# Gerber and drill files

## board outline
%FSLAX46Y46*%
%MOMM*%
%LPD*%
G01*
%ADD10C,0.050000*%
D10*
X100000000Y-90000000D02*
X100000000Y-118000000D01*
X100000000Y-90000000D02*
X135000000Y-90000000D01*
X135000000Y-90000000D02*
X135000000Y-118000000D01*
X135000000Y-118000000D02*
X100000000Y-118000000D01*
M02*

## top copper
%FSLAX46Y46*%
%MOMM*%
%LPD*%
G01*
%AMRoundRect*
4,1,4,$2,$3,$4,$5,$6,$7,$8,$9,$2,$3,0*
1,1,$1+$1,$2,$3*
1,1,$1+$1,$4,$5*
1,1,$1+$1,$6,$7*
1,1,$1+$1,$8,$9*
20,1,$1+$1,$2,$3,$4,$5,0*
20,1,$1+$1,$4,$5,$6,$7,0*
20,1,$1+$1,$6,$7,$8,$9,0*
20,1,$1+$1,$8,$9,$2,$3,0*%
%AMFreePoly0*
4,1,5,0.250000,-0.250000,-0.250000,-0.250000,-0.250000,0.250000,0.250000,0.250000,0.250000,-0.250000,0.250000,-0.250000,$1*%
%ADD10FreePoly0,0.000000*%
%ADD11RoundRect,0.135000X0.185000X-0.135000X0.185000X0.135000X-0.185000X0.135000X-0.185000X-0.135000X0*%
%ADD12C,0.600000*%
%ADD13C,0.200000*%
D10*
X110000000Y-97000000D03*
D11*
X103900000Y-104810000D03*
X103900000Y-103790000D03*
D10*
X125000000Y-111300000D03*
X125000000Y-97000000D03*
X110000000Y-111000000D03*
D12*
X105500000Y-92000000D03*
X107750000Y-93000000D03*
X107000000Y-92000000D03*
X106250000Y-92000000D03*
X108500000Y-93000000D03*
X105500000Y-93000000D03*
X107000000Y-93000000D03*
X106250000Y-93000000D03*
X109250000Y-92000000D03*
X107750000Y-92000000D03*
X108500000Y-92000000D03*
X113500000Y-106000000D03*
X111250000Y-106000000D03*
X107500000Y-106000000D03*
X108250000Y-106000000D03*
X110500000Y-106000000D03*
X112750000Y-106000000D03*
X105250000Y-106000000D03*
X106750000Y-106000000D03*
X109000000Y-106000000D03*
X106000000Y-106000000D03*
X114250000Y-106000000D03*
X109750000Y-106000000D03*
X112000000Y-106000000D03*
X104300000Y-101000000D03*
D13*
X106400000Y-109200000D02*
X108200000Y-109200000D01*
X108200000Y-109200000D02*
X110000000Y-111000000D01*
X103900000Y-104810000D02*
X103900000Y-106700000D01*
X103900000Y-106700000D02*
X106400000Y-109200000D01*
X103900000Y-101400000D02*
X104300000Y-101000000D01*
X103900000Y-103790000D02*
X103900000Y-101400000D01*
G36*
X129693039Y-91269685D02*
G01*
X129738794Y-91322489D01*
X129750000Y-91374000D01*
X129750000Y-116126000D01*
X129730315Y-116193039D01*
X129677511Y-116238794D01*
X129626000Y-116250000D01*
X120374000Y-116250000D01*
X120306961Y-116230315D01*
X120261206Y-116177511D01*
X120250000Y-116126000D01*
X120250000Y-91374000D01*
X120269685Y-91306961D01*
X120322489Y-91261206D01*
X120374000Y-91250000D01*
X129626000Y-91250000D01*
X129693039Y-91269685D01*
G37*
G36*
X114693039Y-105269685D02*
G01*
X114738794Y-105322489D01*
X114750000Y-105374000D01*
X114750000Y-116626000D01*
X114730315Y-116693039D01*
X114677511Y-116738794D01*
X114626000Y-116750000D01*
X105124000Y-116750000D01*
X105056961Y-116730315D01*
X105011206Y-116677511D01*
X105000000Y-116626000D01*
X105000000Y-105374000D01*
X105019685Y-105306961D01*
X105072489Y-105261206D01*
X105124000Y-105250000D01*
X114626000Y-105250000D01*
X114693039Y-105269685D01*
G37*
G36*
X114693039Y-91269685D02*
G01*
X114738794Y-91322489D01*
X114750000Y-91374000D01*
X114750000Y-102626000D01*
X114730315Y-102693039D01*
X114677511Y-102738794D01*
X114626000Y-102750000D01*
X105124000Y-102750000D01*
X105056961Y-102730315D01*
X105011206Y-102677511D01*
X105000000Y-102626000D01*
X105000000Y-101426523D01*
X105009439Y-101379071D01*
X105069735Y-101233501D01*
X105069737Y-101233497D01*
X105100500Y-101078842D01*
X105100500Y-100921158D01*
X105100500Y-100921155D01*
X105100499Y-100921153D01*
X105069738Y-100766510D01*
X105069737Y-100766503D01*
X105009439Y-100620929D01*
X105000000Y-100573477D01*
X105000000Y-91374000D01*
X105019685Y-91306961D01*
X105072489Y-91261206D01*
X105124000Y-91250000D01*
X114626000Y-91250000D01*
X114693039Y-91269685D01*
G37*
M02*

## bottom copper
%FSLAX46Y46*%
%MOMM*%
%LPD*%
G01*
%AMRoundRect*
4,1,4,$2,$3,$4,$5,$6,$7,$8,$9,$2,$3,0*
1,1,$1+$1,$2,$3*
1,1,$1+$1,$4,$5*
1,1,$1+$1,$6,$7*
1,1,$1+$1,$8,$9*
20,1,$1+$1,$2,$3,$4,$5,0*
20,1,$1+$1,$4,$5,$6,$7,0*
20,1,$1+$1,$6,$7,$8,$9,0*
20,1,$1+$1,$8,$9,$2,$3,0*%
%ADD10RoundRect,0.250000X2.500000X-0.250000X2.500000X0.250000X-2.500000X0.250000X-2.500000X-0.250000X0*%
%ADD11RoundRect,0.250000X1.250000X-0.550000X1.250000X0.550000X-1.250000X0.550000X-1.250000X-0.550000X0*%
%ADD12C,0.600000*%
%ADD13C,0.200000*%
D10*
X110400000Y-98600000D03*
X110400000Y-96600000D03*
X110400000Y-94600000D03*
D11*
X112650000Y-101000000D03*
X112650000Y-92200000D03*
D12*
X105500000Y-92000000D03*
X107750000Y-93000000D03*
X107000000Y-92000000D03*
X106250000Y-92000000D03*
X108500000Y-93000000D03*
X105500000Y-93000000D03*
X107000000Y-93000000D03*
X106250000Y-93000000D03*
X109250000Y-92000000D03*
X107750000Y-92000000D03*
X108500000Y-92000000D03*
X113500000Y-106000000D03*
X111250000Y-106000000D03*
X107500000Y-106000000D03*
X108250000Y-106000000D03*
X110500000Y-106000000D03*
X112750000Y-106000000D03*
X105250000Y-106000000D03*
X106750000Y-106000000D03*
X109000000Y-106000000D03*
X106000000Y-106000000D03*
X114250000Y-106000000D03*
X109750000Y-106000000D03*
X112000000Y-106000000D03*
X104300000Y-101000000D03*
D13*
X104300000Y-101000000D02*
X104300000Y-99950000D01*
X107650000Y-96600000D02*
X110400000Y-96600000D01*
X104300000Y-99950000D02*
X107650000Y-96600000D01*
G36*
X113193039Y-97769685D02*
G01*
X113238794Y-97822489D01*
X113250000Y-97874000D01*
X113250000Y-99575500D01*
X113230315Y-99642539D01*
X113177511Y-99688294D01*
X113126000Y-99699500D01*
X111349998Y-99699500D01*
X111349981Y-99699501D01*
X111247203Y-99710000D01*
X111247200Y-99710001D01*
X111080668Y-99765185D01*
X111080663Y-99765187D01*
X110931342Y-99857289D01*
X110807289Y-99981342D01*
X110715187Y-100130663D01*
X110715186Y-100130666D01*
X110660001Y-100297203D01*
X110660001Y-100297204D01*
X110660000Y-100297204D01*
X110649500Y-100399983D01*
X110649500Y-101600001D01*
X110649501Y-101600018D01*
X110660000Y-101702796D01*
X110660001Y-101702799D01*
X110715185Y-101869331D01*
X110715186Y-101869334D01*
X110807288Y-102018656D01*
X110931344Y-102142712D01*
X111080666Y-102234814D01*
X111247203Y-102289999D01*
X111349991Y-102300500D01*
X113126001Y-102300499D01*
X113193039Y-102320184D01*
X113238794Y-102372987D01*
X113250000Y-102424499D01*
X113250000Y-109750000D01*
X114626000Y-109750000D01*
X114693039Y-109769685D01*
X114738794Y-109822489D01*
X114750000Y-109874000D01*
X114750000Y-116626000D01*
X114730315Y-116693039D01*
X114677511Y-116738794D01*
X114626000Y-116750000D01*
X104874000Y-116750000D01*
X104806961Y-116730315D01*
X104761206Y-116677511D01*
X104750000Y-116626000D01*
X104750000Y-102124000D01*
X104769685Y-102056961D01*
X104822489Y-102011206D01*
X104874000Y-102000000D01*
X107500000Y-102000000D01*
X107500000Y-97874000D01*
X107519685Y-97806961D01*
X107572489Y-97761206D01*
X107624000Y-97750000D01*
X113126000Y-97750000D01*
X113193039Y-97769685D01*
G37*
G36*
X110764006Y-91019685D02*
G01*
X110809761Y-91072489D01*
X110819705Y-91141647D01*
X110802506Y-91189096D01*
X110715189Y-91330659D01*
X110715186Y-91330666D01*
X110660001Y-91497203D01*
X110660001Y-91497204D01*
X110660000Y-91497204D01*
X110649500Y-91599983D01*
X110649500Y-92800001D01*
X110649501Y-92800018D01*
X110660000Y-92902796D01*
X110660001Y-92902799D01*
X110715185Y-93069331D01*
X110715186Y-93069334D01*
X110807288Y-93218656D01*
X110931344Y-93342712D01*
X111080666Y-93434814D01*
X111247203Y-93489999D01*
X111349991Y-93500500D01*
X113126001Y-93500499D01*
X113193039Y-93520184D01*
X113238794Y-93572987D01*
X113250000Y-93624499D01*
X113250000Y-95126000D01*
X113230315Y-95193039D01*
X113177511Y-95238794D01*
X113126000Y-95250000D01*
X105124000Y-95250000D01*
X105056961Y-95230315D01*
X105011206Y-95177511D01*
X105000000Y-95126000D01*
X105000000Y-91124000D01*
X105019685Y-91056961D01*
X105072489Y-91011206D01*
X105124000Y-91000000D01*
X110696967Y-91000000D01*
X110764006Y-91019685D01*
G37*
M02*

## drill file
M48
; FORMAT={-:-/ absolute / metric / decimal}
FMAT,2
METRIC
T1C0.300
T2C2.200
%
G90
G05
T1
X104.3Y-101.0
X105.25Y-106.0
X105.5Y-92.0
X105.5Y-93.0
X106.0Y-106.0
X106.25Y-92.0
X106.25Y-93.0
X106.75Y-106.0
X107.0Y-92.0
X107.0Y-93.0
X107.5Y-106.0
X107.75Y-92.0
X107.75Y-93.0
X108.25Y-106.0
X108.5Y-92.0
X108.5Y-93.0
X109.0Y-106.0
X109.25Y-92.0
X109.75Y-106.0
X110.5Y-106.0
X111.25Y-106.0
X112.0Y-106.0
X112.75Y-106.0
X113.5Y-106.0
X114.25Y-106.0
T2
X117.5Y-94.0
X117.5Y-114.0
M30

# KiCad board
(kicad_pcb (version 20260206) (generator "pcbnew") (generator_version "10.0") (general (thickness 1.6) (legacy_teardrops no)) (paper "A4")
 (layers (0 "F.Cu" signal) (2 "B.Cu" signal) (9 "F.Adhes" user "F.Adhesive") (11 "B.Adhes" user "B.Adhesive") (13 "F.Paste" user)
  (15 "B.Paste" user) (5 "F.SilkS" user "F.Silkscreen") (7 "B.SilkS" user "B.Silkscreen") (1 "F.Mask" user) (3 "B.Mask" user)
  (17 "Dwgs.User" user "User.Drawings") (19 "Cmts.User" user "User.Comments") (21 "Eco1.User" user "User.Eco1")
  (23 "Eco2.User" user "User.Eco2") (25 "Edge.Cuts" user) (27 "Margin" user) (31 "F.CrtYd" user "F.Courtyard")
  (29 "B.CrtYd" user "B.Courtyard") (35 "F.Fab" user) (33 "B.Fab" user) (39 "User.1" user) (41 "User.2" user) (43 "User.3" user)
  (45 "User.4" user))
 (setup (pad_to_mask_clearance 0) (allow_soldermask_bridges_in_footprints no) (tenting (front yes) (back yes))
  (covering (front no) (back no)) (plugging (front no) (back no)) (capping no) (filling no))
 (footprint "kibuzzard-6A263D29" (layer "F.Cu") (at 132.5 92.25)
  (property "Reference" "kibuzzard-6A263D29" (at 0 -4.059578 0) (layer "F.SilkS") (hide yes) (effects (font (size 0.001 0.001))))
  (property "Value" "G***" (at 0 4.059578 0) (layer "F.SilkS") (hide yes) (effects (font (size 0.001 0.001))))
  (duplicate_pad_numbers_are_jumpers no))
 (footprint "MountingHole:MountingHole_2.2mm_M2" (layer "F.Cu") (at 117.5 94)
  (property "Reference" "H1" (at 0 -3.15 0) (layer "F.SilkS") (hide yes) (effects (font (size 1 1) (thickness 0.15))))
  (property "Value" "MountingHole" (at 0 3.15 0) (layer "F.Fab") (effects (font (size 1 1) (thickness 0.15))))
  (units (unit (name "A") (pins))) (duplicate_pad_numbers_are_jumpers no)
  (pad "" np_thru_hole circle (at 0 0) (size 2.2 2.2) (drill 2.2) (layers "*.Cu" "*.Mask")))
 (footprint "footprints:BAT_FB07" (layer "F.Cu") (at 110 97)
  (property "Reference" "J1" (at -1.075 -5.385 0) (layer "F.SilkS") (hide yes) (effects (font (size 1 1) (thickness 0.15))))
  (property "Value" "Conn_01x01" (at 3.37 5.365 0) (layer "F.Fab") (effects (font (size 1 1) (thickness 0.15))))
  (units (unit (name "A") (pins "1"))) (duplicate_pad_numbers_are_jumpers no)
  (pad "1" smd custom (at 0 0) (size 0.5 0.5) (layers "F.Cu") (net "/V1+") (options (clearance outline) (anchor rect)) (primitives)))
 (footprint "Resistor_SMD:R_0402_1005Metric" (layer "F.Cu") (at 103.9 104.3 90)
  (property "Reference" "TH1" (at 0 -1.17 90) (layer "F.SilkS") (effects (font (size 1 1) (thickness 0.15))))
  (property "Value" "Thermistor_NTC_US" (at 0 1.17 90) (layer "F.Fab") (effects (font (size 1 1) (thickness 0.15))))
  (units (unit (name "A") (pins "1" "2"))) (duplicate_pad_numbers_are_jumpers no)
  (pad "1" smd roundrect (at -0.51 0 90) (size 0.54 0.64) (layers "F.Cu" "F.Mask" "F.Paste") (roundrect_rratio 0.25) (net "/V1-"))
  (pad "2" smd roundrect (at 0.51 0 90) (size 0.54 0.64) (layers "F.Cu" "F.Mask" "F.Paste") (roundrect_rratio 0.25) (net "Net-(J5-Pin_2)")))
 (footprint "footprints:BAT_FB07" (layer "F.Cu") (at 125 111.3)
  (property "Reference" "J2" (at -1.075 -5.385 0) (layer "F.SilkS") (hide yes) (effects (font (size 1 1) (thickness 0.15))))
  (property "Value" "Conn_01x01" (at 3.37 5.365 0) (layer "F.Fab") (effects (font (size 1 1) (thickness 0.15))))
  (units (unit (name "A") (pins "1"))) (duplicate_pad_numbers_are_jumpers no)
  (pad "1" smd custom (at 0 0) (size 0.5 0.5) (layers "F.Cu") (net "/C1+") (options (clearance outline) (anchor rect)) (primitives)))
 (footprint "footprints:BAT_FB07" (layer "F.Cu") (at 125 97)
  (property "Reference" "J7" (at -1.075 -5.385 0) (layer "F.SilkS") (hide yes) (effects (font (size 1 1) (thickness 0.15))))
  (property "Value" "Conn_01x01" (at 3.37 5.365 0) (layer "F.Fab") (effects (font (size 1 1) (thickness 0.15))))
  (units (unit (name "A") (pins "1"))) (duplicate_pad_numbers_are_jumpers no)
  (pad "1" smd custom (at 0 0) (size 0.5 0.5) (layers "F.Cu") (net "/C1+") (options (clearance outline) (anchor rect)) (primitives)))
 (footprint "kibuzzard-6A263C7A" (layer "F.Cu") (at 102.5 93)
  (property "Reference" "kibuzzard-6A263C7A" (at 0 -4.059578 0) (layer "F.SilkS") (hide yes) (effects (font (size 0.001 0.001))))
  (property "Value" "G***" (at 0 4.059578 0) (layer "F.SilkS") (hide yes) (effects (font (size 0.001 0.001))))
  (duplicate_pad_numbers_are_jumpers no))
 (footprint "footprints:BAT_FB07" (layer "F.Cu") (at 110 111)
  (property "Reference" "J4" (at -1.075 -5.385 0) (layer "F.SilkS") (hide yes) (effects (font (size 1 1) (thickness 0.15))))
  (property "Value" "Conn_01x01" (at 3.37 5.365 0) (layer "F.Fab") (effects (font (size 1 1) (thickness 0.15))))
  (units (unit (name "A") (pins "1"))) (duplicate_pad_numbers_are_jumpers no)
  (pad "1" smd custom (at 0 0) (size 0.5 0.5) (layers "F.Cu") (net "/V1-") (options (clearance outline) (anchor rect)) (primitives)))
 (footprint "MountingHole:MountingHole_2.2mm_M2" (layer "F.Cu") (at 117.5 114)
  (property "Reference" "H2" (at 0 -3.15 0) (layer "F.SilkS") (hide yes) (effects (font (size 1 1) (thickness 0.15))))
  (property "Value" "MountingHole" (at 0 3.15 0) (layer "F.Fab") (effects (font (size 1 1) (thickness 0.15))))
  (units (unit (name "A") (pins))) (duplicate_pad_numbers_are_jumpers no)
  (pad "" np_thru_hole circle (at 0 0) (size 2.2 2.2) (drill 2.2) (layers "*.Cu" "*.Mask")))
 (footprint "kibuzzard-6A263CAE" (layer "F.Cu") (at 102.5 115.25)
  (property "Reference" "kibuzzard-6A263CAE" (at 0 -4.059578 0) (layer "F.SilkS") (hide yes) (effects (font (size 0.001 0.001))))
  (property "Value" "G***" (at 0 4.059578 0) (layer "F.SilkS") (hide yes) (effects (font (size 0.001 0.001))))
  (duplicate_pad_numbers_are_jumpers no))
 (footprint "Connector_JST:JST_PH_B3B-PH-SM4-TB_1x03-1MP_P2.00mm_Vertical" (layer "B.Cu") (at 110.9 96.6 90)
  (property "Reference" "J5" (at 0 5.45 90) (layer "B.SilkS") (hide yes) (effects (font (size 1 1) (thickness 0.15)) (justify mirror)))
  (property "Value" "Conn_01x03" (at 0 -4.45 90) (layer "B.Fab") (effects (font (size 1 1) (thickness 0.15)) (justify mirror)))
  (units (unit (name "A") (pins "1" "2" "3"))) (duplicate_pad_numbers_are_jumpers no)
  (pad "1" smd roundrect (at -2 -0.5 90) (size 1 5.5) (layers "B.Cu" "B.Mask" "B.Paste") (roundrect_rratio 0.25) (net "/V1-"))
  (pad "2" smd roundrect (at 0 -0.5 90) (size 1 5.5) (layers "B.Cu" "B.Mask" "B.Paste") (roundrect_rratio 0.25) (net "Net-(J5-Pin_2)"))
  (pad "3" smd roundrect (at 2 -0.5 90) (size 1 5.5) (layers "B.Cu" "B.Mask" "B.Paste") (roundrect_rratio 0.25) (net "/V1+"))
  (pad "MP" smd roundrect (at -4.4 1.75 90) (size 1.6 3) (layers "B.Cu" "B.Mask" "B.Paste") (roundrect_rratio 0.15625))
  (pad "MP" smd roundrect (at 4.4 1.75 90) (size 1.6 3) (layers "B.Cu" "B.Mask" "B.Paste") (roundrect_rratio 0.15625)))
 (gr_line (start 100 90) (end 100 118) (stroke (width 0.05) (type default)) (layer "Edge.Cuts"))
 (gr_line (start 100 90) (end 135 90) (stroke (width 0.05) (type default)) (layer "Edge.Cuts"))
 (gr_line (start 135 90) (end 135 118) (stroke (width 0.05) (type default)) (layer "Edge.Cuts"))
 (gr_line (start 135 118) (end 100 118) (stroke (width 0.05) (type default)) (layer "Edge.Cuts"))
 (via (at 105.5 92) (size 0.6) (drill 0.3) (layers "F.Cu" "B.Cu") (free yes) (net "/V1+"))
 (via (at 107.75 93) (size 0.6) (drill 0.3) (layers "F.Cu" "B.Cu") (free yes) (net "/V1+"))
 (via (at 107 92) (size 0.6) (drill 0.3) (layers "F.Cu" "B.Cu") (free yes) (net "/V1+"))
 (via (at 106.25 92) (size 0.6) (drill 0.3) (layers "F.Cu" "B.Cu") (free yes) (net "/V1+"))
 (via (at 108.5 93) (size 0.6) (drill 0.3) (layers "F.Cu" "B.Cu") (free yes) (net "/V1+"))
 (via (at 105.5 93) (size 0.6) (drill 0.3) (layers "F.Cu" "B.Cu") (free yes) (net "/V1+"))
 (via (at 107 93) (size 0.6) (drill 0.3) (layers "F.Cu" "B.Cu") (free yes) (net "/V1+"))
 (via (at 106.25 93) (size 0.6) (drill 0.3) (layers "F.Cu" "B.Cu") (free yes) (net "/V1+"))
 (via (at 109.25 92) (size 0.6) (drill 0.3) (layers "F.Cu" "B.Cu") (free yes) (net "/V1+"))
 (via (at 107.75 92) (size 0.6) (drill 0.3) (layers "F.Cu" "B.Cu") (free yes) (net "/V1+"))
 (via (at 108.5 92) (size 0.6) (drill 0.3) (layers "F.Cu" "B.Cu") (free yes) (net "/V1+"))
 (segment (start 106.4 109.2) (end 108.2 109.2) (width 0.2) (layer "F.Cu") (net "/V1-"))
 (segment (start 108.2 109.2) (end 110 111) (width 0.2) (layer "F.Cu") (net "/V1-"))
 (segment (start 103.9 104.81) (end 103.9 106.7) (width 0.2) (layer "F.Cu") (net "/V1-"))
 (segment (start 103.9 106.7) (end 106.4 109.2) (width 0.2) (layer "F.Cu") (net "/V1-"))
 (via (at 113.5 106) (size 0.6) (drill 0.3) (layers "F.Cu" "B.Cu") (free yes) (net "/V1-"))
 (via (at 111.25 106) (size 0.6) (drill 0.3) (layers "F.Cu" "B.Cu") (free yes) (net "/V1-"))
 (via (at 107.5 106) (size 0.6) (drill 0.3) (layers "F.Cu" "B.Cu") (free yes) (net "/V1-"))
 (via (at 108.25 106) (size 0.6) (drill 0.3) (layers "F.Cu" "B.Cu") (free yes) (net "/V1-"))
 (via (at 110.5 106) (size 0.6) (drill 0.3) (layers "F.Cu" "B.Cu") (free yes) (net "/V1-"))
 (via (at 112.75 106) (size 0.6) (drill 0.3) (layers "F.Cu" "B.Cu") (free yes) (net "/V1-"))
 (via (at 105.25 106) (size 0.6) (drill 0.3) (layers "F.Cu" "B.Cu") (free yes) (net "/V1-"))
 (via (at 106.75 106) (size 0.6) (drill 0.3) (layers "F.Cu" "B.Cu") (free yes) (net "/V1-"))
 (via (at 109 106) (size 0.6) (drill 0.3) (layers "F.Cu" "B.Cu") (free yes) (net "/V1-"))
 (via (at 106 106) (size 0.6) (drill 0.3) (layers "F.Cu" "B.Cu") (free yes) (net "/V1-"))
 (via (at 114.25 106) (size 0.6) (drill 0.3) (layers "F.Cu" "B.Cu") (free yes) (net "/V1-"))
 (via (at 109.75 106) (size 0.6) (drill 0.3) (layers "F.Cu" "B.Cu") (free yes) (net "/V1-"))
 (via (at 112 106) (size 0.6) (drill 0.3) (layers "F.Cu" "B.Cu") (free yes) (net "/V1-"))
 (segment (start 103.9 101.4) (end 104.3 101) (width 0.2) (layer "F.Cu") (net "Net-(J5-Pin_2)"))
 (segment (start 103.9 103.79) (end 103.9 101.4) (width 0.2) (layer "F.Cu") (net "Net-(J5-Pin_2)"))
 (via (at 104.3 101) (size 0.6) (drill 0.3) (layers "F.Cu" "B.Cu") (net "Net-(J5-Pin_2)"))
 (segment (start 104.3 101) (end 104.3 99.95) (width 0.2) (layer "B.Cu") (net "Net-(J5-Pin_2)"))
 (segment (start 107.65 96.6) (end 110.4 96.6) (width 0.2) (layer "B.Cu") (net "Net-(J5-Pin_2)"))
 (segment (start 104.3 99.95) (end 107.65 96.6) (width 0.2) (layer "B.Cu") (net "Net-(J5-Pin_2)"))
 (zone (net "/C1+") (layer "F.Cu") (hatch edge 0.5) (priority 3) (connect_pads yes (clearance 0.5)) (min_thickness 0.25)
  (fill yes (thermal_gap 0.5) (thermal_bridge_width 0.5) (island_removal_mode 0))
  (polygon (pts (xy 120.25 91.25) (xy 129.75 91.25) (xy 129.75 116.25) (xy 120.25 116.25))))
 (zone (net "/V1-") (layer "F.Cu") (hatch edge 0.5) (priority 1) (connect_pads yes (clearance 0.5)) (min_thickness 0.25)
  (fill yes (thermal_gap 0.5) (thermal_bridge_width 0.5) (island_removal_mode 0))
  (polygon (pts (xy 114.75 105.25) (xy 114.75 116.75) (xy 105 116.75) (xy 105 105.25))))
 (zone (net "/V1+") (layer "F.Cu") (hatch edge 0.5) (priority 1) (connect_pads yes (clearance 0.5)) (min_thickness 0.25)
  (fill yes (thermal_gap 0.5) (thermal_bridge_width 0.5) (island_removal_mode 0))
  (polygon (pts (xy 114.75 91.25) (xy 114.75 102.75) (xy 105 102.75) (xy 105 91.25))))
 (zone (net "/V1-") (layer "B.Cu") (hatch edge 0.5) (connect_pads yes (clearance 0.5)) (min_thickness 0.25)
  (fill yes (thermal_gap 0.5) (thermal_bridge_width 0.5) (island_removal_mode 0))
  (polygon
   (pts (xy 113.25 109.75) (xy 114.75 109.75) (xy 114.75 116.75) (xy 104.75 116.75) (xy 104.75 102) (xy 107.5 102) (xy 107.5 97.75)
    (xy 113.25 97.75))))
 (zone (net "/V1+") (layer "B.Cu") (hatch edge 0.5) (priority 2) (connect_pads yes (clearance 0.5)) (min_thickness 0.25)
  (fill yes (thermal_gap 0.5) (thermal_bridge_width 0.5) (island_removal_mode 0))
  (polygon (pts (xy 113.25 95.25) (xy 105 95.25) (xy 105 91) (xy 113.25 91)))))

